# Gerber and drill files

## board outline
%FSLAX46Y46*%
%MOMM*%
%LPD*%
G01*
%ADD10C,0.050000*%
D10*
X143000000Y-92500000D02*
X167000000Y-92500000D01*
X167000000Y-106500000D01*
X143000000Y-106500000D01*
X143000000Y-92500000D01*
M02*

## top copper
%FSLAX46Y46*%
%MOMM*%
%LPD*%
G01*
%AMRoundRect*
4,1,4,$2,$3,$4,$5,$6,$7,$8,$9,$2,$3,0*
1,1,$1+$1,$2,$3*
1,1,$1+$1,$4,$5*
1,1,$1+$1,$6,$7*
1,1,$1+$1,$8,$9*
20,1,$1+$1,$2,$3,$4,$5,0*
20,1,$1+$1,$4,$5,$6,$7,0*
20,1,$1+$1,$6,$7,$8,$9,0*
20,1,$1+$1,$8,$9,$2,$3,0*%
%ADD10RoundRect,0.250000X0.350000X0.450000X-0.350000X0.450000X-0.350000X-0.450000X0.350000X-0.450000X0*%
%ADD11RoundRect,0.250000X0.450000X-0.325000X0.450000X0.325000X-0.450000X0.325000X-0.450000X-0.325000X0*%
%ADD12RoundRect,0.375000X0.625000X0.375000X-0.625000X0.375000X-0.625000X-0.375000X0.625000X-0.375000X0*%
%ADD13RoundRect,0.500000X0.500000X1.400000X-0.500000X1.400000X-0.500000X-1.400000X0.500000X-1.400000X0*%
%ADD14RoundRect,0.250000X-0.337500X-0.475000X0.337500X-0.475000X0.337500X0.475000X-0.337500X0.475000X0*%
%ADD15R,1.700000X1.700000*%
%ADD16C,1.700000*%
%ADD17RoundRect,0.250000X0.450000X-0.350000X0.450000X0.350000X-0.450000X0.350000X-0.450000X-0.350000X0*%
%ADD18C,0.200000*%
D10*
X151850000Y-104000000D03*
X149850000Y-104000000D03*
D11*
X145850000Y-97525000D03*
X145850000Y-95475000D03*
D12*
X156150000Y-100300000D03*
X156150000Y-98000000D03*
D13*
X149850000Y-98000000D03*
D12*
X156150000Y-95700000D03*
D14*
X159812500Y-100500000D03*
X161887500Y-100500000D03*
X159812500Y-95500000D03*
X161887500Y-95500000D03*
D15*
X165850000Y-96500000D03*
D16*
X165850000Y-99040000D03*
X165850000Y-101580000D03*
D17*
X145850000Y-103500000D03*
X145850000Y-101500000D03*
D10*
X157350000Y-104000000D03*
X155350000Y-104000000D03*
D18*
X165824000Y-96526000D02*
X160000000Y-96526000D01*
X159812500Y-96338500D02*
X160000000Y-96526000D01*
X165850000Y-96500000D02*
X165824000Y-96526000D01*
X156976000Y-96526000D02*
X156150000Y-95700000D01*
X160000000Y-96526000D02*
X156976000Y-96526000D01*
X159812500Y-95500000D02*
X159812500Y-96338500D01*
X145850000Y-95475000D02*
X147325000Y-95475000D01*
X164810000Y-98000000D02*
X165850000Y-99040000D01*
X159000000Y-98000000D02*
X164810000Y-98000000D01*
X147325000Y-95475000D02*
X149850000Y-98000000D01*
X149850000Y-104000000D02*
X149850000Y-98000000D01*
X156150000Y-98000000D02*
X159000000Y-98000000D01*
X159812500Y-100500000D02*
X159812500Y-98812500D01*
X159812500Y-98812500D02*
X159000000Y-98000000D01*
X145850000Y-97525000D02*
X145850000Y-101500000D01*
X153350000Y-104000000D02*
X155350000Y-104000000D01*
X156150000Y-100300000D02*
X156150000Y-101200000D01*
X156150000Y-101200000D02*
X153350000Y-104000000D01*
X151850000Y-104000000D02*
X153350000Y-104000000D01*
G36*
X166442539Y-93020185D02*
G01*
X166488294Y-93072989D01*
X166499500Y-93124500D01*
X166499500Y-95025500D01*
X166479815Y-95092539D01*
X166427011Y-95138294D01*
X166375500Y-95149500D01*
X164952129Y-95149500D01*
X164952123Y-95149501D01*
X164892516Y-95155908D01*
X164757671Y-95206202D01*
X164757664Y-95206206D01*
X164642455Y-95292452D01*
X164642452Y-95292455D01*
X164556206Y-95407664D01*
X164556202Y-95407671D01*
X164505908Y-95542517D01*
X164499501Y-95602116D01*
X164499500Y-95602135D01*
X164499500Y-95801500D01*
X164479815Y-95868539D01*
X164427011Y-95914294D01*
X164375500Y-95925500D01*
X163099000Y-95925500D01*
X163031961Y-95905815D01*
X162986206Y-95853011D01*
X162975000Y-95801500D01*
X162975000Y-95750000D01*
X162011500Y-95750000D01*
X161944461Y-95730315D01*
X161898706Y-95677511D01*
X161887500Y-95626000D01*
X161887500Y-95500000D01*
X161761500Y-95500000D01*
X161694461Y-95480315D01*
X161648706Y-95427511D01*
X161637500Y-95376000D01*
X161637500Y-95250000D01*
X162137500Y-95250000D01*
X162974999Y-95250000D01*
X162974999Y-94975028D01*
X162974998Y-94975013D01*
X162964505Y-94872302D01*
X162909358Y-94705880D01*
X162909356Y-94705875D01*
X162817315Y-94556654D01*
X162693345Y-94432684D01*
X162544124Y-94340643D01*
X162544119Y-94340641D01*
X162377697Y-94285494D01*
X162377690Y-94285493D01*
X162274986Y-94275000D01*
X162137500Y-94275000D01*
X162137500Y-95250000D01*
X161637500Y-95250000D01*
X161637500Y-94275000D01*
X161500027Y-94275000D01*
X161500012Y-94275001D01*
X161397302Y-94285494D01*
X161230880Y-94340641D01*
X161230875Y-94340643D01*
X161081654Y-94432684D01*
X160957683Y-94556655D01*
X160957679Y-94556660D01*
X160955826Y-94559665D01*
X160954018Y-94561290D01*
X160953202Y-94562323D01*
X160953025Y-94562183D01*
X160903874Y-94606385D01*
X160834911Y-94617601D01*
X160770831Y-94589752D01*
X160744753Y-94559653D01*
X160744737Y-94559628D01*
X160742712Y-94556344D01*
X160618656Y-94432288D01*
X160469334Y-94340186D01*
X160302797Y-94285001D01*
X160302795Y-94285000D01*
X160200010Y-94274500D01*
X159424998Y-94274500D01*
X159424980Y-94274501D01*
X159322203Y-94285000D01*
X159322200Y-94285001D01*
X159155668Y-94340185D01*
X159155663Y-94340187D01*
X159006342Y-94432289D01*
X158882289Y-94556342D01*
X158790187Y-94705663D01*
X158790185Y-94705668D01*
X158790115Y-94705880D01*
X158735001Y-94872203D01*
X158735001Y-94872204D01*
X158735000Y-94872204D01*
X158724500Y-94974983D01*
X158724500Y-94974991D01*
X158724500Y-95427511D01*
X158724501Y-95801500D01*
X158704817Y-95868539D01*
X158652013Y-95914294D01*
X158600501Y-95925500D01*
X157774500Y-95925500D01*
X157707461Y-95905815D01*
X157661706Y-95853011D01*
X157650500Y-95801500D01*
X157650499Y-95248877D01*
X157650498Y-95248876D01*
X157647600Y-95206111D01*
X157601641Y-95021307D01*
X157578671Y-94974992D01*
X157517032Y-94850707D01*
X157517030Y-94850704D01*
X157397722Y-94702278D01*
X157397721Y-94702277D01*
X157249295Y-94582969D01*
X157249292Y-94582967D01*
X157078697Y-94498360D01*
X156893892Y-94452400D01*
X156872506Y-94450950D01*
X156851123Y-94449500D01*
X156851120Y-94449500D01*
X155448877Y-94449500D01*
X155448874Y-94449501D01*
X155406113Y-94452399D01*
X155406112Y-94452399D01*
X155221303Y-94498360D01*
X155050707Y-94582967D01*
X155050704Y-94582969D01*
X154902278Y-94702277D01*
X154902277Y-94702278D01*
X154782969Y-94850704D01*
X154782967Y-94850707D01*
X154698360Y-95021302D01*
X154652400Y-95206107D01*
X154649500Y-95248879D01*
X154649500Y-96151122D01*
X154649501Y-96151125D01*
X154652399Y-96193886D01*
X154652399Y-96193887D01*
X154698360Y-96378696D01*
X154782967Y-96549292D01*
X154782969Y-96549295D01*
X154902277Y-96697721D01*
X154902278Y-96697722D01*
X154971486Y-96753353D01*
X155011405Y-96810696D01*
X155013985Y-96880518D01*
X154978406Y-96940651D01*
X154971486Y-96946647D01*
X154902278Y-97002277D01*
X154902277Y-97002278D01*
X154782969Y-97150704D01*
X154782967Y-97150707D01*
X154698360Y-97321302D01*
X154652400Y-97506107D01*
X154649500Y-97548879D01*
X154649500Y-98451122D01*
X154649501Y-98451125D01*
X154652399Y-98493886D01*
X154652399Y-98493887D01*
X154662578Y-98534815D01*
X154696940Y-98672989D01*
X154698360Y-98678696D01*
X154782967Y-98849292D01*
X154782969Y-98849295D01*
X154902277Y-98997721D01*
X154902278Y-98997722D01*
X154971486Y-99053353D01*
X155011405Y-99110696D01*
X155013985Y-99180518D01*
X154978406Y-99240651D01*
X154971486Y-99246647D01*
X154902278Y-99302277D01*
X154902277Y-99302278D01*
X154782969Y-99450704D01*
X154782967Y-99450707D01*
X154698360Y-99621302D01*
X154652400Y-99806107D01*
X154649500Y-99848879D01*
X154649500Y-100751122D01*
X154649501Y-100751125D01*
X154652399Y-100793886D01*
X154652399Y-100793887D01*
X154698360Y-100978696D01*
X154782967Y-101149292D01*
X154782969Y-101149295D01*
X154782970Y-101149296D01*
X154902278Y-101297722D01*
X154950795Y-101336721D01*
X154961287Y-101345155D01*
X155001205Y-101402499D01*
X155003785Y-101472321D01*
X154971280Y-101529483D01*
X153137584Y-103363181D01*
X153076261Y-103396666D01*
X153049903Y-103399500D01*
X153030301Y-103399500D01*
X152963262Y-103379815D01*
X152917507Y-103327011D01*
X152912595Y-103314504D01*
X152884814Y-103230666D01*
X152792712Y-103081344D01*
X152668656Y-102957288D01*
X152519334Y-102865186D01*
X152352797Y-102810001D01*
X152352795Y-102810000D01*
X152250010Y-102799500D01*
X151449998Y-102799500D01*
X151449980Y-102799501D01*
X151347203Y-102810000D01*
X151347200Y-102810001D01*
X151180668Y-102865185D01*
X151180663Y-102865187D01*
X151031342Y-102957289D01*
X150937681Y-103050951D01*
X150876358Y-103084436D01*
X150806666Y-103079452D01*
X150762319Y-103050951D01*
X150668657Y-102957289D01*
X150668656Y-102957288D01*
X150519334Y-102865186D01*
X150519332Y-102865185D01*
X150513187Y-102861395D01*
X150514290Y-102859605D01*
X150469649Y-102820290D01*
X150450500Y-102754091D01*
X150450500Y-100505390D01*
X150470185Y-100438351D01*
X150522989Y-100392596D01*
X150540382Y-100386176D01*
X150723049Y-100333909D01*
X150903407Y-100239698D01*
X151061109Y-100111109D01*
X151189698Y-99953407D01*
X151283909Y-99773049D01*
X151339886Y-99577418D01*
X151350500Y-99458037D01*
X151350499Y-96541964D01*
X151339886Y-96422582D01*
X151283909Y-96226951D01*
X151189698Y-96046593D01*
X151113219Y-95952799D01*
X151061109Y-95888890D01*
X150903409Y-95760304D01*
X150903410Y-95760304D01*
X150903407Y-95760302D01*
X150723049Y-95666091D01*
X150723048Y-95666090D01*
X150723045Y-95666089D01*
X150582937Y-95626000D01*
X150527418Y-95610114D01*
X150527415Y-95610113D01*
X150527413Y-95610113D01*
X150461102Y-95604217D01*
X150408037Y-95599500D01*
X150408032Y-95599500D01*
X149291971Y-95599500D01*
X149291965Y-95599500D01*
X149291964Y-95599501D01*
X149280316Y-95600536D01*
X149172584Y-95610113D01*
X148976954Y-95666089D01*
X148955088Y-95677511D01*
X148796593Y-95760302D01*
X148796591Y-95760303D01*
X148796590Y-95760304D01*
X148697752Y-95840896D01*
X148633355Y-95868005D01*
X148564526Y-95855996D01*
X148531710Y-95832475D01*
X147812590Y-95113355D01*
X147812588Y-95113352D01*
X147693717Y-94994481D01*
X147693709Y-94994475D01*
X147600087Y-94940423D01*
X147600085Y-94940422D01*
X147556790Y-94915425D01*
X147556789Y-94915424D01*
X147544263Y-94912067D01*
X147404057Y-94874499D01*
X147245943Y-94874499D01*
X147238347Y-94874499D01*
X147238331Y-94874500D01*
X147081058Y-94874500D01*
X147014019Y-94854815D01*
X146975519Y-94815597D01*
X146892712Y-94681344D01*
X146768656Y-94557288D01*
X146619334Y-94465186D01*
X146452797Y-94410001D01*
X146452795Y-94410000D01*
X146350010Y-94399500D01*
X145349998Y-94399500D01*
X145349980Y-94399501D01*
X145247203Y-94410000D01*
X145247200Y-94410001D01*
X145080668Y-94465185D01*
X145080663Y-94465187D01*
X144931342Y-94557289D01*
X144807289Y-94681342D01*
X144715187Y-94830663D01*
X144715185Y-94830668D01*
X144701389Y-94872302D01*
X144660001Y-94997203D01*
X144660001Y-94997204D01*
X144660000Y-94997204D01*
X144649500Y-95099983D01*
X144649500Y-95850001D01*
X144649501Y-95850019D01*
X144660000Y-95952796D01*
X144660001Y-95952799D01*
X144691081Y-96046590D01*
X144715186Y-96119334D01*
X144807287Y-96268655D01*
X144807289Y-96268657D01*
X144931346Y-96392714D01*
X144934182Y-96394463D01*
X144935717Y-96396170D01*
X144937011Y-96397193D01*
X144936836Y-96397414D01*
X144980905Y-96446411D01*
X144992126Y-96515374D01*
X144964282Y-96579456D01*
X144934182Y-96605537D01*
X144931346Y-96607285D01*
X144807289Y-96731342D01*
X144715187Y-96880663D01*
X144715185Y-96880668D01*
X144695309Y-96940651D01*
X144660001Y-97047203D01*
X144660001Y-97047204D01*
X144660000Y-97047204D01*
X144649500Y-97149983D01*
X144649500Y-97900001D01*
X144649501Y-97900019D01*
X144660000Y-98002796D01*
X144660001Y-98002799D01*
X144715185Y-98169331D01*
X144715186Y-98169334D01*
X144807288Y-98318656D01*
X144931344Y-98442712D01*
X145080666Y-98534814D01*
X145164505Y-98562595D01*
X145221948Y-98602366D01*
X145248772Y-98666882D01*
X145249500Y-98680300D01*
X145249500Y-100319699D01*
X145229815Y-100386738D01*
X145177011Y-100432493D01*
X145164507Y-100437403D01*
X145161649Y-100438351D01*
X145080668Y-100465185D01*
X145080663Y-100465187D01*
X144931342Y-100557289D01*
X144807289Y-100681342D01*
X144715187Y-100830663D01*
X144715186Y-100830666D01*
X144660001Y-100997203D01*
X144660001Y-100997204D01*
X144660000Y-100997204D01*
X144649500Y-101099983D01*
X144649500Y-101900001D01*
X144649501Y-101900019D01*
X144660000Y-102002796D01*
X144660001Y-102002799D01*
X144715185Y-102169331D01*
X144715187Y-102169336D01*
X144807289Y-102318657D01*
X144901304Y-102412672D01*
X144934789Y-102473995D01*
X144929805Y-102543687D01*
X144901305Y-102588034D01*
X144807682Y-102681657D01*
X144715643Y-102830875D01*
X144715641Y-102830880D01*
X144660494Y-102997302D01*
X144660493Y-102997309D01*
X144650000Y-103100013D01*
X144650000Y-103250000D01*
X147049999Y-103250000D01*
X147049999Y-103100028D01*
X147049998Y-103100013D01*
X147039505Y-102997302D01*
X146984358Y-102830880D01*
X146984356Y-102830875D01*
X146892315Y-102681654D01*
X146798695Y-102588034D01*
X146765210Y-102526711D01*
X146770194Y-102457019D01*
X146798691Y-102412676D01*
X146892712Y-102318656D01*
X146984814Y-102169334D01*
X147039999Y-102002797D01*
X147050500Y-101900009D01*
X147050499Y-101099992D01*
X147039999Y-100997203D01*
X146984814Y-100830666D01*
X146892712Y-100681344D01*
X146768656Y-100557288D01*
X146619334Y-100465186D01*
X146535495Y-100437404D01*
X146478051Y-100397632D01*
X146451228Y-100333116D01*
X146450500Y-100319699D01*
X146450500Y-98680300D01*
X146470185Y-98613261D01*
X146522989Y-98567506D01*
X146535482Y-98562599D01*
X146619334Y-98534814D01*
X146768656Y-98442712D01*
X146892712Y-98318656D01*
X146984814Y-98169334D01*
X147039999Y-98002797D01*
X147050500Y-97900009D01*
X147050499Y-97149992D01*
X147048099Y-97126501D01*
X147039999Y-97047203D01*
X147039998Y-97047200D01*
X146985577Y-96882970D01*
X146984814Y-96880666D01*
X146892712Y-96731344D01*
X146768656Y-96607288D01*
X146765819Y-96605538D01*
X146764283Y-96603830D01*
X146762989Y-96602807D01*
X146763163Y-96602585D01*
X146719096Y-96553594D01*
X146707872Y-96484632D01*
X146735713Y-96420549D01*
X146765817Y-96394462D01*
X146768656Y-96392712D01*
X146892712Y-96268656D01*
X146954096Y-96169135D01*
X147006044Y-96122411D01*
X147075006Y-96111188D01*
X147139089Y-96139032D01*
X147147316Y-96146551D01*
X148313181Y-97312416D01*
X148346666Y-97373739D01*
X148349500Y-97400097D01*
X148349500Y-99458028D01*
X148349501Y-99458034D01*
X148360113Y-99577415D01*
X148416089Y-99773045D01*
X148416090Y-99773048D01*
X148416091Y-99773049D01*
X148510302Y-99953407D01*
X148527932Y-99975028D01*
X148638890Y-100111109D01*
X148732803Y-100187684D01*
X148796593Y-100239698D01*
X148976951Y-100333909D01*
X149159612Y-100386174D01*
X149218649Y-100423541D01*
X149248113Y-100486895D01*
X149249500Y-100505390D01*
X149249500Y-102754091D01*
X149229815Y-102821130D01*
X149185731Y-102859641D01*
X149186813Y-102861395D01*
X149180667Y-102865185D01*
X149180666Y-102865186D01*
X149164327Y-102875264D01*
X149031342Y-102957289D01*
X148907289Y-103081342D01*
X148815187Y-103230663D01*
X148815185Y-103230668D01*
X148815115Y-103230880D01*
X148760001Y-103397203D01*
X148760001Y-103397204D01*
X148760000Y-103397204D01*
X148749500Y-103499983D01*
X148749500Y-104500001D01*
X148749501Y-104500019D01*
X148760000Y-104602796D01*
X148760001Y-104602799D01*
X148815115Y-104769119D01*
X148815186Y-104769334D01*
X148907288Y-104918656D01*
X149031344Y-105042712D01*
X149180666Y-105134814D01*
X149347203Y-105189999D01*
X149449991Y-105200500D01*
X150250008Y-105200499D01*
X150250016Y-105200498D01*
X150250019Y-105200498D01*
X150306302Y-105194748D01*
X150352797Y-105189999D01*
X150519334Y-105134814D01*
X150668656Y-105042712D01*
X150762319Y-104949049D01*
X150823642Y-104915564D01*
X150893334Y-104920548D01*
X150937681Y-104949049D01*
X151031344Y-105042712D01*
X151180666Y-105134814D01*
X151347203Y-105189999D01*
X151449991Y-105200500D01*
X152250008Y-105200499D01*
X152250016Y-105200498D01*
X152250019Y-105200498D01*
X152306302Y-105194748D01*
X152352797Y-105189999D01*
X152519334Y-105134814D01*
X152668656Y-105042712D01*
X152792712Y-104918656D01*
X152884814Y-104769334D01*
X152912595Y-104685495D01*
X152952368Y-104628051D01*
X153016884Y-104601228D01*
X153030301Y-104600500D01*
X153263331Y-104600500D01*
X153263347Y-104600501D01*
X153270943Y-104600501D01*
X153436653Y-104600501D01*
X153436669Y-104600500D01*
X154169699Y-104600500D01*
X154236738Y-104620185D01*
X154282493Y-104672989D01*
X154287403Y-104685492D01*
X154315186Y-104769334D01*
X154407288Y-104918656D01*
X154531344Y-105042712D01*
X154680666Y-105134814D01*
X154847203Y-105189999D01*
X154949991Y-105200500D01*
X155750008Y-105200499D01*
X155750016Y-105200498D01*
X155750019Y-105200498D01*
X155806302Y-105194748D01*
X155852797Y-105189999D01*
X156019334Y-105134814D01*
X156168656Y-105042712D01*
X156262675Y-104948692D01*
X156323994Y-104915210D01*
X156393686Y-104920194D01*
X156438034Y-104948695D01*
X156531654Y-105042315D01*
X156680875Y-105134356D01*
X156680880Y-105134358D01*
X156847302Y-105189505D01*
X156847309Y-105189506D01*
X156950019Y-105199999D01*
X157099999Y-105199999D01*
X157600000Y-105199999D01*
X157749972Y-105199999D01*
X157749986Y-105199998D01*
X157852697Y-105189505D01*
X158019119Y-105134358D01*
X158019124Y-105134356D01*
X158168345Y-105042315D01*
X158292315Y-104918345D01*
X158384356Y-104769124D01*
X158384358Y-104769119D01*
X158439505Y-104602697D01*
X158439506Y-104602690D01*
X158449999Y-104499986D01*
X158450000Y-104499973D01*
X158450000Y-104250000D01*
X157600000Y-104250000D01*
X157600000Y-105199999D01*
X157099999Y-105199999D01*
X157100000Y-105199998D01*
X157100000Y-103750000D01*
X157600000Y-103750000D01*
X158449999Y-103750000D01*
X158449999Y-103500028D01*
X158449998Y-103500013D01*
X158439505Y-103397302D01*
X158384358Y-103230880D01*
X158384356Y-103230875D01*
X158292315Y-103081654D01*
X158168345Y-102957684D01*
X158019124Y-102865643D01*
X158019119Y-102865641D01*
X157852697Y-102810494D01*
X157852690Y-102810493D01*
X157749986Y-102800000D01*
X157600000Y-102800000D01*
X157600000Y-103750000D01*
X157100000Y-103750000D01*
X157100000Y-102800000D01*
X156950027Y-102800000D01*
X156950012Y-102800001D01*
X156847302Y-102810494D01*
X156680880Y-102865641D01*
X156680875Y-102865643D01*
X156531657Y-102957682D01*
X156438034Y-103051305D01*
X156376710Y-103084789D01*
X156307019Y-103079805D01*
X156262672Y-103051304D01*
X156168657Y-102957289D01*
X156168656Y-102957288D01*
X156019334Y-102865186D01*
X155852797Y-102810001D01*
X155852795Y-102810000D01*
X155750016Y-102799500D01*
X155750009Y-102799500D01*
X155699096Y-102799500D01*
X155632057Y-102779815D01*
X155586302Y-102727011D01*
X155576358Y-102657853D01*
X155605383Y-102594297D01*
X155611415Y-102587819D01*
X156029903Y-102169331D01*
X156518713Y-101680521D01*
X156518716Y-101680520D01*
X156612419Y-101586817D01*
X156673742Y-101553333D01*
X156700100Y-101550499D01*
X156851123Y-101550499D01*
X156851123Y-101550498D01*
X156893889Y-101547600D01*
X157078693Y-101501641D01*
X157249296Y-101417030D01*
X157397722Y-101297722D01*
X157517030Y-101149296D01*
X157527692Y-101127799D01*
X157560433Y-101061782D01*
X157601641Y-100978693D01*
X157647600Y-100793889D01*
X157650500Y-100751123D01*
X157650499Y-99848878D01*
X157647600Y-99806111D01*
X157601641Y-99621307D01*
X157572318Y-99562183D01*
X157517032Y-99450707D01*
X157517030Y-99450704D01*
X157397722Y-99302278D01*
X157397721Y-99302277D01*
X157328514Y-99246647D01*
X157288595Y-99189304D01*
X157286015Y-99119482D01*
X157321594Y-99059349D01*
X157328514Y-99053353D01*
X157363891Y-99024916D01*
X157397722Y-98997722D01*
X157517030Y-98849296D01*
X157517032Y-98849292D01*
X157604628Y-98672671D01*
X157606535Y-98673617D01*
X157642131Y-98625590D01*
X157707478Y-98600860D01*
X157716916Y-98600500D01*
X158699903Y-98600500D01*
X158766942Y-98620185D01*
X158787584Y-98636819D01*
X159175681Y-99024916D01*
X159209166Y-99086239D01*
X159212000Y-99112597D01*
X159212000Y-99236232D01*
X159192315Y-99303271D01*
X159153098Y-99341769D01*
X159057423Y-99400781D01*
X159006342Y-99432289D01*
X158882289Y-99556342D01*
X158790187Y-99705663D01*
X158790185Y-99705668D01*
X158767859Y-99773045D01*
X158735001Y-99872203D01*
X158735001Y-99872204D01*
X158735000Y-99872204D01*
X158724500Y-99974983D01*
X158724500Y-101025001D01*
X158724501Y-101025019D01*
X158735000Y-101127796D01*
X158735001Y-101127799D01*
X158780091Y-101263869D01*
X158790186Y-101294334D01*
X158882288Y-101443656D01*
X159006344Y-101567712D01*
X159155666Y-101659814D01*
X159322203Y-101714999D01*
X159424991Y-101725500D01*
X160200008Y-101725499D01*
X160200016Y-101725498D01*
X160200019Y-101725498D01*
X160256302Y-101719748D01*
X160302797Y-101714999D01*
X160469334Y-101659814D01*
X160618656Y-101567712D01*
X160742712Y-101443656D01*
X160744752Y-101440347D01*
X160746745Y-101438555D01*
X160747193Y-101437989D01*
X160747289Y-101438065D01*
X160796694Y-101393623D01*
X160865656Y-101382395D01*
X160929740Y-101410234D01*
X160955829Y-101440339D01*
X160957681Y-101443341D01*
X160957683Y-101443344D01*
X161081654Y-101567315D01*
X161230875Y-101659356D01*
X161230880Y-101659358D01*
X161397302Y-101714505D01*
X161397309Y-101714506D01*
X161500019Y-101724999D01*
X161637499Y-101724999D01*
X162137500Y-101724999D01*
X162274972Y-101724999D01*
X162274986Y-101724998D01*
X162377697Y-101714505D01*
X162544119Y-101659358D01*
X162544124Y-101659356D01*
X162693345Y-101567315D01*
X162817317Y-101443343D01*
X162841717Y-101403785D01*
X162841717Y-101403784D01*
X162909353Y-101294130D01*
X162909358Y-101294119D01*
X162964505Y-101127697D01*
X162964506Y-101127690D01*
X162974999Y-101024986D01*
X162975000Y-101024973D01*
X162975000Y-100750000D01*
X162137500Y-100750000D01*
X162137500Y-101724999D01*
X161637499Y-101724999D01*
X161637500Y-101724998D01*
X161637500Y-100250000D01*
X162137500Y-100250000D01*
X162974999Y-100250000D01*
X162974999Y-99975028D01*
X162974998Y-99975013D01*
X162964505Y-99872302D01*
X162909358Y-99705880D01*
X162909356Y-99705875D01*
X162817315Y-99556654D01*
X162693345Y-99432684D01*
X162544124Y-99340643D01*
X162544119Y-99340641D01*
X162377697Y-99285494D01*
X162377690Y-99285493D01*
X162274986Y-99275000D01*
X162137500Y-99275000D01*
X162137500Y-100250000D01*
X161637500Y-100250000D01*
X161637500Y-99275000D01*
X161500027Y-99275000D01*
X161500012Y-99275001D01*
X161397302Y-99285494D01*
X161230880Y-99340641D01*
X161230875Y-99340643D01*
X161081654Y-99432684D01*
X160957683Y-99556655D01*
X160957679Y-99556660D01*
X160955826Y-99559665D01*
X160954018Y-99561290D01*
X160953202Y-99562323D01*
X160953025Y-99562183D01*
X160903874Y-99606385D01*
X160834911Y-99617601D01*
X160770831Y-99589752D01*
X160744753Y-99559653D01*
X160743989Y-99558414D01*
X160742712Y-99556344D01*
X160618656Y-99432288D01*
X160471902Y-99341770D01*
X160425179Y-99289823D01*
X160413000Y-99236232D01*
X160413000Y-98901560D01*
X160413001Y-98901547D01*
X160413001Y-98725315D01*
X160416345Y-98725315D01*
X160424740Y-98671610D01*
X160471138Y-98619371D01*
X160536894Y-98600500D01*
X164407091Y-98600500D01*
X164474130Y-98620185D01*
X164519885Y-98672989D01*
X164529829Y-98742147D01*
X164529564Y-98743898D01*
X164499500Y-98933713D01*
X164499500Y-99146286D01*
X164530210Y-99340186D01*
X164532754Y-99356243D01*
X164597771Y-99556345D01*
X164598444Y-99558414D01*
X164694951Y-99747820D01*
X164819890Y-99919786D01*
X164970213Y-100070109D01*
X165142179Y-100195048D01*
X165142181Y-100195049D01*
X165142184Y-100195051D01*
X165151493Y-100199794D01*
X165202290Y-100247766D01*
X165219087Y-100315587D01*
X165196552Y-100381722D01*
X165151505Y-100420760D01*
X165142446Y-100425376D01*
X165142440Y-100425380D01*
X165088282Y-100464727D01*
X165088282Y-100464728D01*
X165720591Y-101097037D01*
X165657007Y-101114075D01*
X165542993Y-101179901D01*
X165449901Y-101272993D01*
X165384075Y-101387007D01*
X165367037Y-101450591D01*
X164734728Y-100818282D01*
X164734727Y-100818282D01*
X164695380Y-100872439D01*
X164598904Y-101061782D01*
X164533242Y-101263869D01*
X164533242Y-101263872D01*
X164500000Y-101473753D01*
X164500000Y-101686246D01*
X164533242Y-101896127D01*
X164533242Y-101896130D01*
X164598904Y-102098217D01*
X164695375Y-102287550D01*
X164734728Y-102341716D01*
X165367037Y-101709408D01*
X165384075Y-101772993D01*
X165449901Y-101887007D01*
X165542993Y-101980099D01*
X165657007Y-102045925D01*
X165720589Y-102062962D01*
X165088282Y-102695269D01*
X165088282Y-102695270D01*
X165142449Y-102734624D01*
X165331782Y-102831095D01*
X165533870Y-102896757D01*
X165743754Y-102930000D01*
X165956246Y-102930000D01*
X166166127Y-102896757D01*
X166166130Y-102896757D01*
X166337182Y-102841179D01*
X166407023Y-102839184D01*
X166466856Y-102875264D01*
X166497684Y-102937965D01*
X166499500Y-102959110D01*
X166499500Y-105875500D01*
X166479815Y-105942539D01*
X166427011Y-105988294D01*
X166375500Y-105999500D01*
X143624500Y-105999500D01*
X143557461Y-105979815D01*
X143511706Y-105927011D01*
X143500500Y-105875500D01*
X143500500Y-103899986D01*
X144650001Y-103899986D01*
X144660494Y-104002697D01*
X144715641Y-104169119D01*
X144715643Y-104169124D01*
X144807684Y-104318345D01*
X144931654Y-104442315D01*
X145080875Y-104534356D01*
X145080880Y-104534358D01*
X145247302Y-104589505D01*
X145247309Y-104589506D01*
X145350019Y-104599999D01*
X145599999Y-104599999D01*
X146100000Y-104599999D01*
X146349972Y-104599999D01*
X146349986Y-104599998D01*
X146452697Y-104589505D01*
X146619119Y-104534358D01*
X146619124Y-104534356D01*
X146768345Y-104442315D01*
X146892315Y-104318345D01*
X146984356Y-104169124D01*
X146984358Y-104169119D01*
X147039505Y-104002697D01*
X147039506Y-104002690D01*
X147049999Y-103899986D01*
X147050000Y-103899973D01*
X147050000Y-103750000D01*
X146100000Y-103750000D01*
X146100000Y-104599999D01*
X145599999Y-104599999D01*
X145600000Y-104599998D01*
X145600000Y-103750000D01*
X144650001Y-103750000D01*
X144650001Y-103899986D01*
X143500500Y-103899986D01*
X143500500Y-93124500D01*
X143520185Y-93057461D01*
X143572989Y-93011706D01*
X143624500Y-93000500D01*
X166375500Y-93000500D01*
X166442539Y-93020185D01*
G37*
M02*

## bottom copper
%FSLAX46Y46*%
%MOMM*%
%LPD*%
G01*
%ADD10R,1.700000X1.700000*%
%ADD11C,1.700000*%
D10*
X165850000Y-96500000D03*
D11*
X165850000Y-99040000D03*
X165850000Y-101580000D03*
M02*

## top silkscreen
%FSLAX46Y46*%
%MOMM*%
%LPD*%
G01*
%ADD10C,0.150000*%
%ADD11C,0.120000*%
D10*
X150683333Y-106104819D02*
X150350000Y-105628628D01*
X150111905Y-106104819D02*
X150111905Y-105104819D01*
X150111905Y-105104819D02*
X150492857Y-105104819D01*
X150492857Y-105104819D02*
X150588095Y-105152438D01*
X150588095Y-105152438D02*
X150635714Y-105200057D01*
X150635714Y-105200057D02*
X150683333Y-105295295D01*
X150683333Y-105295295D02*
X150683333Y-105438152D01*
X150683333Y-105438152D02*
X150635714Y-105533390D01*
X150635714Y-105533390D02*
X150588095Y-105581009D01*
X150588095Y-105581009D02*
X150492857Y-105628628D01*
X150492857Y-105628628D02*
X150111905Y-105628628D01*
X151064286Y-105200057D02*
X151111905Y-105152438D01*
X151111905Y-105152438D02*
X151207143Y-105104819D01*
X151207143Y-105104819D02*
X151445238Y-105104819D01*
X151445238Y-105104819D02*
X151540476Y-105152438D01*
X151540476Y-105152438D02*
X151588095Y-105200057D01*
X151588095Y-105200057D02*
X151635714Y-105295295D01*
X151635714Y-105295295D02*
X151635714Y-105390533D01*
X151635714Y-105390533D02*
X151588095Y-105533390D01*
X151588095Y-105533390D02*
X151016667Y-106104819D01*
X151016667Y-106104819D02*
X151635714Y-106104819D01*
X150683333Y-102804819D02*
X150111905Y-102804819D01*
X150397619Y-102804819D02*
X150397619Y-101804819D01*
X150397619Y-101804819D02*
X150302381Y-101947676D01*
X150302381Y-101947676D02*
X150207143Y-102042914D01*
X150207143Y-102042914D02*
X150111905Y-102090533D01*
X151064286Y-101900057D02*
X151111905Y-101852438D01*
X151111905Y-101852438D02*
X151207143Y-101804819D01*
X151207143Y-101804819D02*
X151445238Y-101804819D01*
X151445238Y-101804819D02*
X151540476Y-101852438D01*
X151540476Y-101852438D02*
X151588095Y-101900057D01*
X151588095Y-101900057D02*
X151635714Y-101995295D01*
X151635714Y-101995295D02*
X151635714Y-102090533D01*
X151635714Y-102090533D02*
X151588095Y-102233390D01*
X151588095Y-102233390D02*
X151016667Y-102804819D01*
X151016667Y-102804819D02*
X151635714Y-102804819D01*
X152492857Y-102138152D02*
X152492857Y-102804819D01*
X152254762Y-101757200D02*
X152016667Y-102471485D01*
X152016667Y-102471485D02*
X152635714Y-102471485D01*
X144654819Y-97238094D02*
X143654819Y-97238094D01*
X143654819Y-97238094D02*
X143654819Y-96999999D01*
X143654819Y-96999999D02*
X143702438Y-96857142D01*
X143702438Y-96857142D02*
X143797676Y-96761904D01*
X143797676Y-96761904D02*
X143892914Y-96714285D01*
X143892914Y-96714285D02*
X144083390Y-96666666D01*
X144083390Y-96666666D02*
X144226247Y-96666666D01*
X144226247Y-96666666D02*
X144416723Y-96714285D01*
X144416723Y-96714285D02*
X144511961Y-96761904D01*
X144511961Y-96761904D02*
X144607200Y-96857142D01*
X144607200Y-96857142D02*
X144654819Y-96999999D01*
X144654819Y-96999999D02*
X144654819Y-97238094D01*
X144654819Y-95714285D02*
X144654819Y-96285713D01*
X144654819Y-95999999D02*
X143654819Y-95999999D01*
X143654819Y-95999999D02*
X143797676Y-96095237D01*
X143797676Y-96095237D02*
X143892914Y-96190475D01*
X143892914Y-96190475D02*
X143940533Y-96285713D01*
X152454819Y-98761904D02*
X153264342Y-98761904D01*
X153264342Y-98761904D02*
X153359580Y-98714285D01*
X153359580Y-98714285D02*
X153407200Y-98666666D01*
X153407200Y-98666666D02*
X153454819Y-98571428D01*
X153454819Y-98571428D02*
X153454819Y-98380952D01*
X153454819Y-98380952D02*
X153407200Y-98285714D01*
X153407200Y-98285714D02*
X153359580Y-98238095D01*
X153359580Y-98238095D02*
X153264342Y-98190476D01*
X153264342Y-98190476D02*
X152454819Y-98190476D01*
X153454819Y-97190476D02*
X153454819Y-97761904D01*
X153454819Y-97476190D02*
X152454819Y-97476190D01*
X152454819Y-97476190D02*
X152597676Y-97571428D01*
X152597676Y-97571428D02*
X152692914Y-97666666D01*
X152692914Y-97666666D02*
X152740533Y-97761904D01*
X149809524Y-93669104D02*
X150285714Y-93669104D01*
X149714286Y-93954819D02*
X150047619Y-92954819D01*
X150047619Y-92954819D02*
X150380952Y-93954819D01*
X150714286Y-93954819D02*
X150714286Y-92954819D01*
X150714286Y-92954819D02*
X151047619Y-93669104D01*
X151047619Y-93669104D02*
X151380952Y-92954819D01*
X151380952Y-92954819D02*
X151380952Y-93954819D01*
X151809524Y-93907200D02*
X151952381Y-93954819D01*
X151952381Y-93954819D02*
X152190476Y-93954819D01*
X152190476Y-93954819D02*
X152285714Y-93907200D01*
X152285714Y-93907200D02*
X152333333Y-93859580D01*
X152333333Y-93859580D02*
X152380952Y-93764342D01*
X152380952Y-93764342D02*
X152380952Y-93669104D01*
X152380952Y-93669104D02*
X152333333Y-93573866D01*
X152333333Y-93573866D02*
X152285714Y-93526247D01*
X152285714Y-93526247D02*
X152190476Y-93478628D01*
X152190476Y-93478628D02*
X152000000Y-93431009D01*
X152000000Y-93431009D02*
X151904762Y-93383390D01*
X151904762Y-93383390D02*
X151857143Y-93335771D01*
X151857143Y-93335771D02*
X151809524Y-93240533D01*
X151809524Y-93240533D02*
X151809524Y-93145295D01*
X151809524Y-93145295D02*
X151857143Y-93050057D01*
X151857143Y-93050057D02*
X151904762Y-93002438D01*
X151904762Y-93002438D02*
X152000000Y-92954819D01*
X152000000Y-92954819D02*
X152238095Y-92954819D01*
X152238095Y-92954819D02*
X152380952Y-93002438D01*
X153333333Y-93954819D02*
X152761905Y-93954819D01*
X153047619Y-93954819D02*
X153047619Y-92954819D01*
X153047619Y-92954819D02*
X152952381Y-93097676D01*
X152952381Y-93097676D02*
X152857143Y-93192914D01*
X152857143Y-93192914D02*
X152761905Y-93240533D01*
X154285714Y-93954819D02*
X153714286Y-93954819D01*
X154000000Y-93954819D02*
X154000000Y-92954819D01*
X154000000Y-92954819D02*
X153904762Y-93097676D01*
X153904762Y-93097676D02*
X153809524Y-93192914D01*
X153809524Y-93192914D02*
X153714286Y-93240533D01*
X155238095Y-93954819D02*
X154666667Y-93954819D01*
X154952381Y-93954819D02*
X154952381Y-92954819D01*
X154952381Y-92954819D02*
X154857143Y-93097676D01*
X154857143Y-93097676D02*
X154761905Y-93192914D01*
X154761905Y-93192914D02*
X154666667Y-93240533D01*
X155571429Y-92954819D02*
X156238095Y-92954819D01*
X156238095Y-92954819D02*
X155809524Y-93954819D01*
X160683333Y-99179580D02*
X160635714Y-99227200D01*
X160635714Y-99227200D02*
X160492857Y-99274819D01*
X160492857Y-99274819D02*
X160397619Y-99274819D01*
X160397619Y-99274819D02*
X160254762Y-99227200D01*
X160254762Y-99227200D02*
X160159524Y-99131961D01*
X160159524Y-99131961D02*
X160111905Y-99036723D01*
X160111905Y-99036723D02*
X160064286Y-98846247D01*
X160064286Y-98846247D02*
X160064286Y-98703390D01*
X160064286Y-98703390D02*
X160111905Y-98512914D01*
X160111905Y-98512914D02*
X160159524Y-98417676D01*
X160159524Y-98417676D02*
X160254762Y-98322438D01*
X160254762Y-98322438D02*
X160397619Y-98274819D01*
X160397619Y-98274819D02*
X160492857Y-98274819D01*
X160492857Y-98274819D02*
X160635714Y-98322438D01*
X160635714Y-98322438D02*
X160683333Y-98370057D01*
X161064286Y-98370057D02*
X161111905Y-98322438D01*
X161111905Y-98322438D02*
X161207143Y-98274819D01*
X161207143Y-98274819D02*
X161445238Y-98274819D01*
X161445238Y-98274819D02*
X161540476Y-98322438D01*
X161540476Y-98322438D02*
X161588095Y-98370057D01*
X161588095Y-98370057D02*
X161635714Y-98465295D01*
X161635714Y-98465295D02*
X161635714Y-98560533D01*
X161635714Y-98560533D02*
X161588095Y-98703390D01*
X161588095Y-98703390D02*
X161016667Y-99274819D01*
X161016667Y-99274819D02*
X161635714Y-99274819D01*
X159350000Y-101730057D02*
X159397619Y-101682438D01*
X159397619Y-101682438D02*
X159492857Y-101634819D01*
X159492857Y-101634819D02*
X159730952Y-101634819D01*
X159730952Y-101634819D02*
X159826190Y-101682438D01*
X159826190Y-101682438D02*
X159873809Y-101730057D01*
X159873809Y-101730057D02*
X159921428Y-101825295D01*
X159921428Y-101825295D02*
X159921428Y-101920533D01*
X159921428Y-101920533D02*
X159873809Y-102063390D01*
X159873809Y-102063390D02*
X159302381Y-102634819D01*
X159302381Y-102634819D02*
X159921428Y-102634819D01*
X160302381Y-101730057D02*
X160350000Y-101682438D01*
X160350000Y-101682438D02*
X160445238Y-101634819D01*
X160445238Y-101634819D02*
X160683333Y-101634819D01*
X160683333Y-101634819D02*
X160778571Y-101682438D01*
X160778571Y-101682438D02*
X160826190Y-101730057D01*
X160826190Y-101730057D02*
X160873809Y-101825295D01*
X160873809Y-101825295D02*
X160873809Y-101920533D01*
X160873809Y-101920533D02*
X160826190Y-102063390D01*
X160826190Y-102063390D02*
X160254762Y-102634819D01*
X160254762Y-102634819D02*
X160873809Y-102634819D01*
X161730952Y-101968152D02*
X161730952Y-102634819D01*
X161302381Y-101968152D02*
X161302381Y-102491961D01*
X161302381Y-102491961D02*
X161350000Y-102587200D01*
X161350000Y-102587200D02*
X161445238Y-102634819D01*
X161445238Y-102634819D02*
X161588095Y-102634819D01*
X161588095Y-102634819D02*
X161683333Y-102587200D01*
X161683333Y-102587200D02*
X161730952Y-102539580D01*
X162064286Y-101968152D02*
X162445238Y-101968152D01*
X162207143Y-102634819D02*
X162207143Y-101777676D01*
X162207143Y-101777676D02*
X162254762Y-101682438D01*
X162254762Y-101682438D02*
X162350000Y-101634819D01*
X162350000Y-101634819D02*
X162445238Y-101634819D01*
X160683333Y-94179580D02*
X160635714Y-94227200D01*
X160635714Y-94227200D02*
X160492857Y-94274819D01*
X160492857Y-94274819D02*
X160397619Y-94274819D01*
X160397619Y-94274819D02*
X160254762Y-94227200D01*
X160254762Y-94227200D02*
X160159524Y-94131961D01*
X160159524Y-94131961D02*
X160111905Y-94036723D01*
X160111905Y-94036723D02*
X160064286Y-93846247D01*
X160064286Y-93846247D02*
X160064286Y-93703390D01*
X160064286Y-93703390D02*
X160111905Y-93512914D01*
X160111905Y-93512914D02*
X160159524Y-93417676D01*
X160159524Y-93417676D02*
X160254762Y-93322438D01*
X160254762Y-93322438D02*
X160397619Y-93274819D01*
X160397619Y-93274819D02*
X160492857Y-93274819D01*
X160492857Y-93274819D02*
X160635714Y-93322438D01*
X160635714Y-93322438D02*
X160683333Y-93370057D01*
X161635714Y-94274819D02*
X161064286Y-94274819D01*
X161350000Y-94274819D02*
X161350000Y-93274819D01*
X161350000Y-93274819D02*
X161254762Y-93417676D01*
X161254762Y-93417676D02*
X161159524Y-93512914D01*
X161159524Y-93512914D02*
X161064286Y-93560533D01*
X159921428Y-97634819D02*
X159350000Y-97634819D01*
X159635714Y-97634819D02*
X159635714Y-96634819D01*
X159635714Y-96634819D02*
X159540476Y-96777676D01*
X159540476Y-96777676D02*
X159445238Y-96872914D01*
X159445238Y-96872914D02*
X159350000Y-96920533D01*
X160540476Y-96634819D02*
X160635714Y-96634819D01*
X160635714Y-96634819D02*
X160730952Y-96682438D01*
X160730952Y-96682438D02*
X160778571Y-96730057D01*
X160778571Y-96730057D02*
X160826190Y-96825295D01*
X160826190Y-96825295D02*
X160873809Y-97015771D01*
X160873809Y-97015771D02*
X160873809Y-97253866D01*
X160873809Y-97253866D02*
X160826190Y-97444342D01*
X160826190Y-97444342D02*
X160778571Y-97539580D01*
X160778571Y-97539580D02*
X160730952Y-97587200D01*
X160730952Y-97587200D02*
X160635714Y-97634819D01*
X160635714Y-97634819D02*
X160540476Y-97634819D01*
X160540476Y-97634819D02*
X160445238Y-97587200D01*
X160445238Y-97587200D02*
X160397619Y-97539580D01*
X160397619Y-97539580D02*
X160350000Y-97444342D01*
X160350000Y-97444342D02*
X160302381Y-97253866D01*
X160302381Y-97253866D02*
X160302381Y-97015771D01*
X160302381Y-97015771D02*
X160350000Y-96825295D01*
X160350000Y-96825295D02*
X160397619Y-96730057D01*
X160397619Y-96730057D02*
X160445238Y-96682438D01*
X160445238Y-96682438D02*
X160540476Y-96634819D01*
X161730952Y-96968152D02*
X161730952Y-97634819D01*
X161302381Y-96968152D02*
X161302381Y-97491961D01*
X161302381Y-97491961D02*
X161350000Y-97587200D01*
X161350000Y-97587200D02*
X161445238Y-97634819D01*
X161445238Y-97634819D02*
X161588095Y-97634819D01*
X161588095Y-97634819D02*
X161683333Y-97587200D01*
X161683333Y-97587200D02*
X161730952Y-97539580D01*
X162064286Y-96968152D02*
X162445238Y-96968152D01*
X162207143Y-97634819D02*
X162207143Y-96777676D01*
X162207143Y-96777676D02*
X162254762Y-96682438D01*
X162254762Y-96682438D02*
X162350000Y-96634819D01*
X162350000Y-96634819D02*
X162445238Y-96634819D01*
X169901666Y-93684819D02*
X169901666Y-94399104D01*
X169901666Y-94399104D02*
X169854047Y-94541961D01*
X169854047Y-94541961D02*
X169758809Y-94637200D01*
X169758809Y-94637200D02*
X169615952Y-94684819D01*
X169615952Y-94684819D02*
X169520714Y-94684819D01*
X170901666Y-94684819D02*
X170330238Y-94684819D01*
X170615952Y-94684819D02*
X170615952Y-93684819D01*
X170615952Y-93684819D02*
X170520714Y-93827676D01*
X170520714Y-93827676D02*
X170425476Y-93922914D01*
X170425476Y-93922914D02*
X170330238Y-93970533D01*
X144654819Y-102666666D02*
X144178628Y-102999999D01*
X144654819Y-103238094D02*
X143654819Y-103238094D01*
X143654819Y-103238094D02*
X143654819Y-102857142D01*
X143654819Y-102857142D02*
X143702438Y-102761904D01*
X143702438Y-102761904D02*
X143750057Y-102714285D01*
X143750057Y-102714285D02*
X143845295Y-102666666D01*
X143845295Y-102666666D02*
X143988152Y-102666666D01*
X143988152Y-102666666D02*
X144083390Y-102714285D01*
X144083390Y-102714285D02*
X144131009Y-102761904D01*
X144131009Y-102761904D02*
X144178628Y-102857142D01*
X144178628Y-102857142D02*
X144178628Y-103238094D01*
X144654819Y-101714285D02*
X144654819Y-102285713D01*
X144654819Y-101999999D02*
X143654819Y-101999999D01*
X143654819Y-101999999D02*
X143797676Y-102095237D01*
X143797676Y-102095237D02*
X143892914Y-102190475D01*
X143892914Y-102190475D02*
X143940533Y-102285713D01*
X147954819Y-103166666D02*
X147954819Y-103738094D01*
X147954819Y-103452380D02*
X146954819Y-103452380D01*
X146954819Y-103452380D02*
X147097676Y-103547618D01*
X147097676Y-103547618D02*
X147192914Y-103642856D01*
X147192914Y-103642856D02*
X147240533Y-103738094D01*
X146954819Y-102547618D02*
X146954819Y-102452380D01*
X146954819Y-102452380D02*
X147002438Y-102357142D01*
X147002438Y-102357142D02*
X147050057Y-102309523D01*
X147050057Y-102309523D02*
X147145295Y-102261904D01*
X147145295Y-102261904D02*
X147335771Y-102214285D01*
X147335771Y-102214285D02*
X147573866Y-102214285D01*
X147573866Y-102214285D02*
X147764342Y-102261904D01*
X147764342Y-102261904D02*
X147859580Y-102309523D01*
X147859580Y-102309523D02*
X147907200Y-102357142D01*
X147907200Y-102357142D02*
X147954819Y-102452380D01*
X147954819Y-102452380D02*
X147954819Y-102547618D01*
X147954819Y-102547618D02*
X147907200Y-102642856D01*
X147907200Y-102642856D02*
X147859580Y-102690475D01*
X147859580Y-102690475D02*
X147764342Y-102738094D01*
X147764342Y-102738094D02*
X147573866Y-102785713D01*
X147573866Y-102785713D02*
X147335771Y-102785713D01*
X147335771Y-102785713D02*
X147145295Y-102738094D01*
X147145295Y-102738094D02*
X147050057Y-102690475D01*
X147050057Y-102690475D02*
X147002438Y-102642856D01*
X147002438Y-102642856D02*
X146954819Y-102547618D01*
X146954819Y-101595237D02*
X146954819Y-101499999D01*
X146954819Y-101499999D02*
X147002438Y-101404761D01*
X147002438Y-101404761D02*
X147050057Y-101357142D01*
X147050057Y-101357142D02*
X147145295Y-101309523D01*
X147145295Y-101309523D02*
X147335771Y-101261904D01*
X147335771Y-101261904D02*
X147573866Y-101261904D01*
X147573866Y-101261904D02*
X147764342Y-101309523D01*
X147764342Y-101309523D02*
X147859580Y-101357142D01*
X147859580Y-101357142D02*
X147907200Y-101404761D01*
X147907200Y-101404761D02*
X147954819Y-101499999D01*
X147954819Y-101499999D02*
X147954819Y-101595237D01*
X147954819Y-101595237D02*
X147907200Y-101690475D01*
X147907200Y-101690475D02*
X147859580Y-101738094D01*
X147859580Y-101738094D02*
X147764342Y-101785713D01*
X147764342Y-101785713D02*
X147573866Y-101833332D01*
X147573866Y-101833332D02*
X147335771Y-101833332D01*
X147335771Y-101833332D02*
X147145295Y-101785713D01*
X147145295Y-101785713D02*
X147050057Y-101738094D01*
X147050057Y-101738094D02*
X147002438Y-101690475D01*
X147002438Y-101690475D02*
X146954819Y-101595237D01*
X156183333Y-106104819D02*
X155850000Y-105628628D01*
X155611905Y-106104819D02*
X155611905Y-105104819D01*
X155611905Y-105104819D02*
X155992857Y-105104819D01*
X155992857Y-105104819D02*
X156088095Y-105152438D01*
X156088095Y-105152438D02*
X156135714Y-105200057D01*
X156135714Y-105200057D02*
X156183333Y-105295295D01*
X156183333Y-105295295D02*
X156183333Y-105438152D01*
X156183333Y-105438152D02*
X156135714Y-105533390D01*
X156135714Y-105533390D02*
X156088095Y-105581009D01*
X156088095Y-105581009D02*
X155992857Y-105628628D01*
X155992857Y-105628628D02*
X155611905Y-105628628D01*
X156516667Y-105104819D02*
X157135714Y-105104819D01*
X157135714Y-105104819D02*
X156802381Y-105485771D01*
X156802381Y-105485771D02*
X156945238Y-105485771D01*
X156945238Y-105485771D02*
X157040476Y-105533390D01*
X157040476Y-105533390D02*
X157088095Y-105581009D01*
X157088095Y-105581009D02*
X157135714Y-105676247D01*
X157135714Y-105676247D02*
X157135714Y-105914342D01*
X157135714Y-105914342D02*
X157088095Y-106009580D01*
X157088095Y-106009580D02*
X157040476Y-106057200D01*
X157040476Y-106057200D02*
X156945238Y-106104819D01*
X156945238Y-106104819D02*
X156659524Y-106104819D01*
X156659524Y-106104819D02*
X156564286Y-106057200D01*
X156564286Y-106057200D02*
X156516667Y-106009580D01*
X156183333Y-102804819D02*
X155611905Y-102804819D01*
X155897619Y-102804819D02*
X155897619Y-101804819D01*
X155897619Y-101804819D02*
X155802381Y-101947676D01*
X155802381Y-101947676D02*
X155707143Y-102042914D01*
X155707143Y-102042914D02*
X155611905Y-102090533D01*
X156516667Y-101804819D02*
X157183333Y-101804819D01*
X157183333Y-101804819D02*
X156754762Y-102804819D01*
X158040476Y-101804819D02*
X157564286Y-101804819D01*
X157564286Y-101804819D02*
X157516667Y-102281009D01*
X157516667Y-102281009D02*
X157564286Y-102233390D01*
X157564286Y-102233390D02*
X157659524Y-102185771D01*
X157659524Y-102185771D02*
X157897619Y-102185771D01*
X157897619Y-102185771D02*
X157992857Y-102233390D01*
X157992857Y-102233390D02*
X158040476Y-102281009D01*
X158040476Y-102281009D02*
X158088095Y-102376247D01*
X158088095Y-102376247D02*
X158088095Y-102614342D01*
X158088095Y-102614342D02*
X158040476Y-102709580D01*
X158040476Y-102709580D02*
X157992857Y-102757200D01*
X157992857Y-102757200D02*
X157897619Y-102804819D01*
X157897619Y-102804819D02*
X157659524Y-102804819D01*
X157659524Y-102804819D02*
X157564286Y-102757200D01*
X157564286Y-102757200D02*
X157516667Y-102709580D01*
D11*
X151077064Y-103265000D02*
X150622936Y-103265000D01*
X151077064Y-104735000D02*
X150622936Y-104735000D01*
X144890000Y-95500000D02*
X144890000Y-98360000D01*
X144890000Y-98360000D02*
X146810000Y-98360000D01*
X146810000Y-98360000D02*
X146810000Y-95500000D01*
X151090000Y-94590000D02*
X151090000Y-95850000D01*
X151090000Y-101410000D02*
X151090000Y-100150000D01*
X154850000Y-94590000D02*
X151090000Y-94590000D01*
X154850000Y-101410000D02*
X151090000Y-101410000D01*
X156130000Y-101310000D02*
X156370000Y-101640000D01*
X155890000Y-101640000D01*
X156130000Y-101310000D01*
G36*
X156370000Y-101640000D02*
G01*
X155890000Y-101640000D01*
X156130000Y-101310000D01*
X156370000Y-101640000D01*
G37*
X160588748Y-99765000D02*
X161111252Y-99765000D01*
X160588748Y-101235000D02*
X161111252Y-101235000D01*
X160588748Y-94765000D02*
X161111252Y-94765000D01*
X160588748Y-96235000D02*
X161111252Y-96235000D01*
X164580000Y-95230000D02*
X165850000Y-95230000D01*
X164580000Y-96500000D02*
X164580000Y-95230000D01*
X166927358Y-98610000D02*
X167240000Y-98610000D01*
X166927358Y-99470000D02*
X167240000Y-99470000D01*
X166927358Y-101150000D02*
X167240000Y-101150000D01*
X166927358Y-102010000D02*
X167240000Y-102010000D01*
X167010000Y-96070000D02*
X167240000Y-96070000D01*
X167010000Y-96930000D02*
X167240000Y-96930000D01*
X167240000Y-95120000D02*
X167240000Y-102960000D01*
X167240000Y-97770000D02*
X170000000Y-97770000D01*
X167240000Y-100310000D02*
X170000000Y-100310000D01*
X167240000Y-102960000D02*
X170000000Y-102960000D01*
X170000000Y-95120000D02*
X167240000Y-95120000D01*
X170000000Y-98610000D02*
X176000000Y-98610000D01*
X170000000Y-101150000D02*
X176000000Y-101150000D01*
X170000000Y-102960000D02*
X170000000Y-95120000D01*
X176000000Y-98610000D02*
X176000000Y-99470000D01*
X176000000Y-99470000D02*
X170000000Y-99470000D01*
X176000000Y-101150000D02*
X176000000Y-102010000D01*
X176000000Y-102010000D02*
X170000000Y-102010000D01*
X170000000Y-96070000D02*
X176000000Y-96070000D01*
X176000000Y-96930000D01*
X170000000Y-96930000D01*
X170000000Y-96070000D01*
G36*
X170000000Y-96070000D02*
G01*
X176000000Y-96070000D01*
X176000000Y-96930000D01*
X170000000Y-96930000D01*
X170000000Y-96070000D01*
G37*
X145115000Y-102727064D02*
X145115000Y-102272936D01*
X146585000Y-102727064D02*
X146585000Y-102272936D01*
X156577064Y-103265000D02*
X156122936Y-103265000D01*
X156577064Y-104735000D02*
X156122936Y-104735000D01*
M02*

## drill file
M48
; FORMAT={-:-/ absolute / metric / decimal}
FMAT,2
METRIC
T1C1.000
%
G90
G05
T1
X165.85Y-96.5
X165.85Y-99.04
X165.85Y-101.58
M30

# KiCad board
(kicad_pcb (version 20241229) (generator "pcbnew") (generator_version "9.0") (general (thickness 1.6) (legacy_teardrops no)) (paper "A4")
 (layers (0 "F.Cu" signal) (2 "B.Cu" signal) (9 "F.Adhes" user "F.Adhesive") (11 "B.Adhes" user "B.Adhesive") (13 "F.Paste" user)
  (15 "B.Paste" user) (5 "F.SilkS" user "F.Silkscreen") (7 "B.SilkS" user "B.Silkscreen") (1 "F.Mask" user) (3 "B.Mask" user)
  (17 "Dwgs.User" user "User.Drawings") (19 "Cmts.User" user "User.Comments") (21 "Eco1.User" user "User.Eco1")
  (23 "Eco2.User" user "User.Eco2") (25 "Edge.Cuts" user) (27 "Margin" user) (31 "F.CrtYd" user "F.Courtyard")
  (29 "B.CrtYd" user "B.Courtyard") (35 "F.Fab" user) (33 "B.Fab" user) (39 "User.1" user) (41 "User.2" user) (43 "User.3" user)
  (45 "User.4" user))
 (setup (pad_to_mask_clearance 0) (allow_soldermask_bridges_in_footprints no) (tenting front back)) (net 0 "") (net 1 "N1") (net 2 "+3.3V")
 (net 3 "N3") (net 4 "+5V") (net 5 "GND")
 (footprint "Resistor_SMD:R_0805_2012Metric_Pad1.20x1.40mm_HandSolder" (layer "F.Cu") (at 150.85 104 180)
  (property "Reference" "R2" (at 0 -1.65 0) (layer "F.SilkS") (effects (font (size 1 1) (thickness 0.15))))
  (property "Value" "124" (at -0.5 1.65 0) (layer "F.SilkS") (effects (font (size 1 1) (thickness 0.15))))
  (fp_line (start -0.227064 0.735) (end 0.227064 0.735) (stroke (width 0.12) (type solid)) (layer "F.SilkS"))
  (fp_line (start -0.227064 -0.735) (end 0.227064 -0.735) (stroke (width 0.12) (type solid)) (layer "F.SilkS"))
  (pad "1" smd roundrect (at -1 0 180) (size 1.2 1.4) (layers "F.Cu" "F.Mask" "F.Paste") (roundrect_rratio 0.208333) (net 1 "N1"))
  (pad "2" smd roundrect (at 1 0 180) (size 1.2 1.4) (layers "F.Cu" "F.Mask" "F.Paste") (roundrect_rratio 0.208333) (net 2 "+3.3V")))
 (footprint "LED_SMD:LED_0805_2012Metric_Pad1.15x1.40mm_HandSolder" (layer "F.Cu") (at 145.85 96.5 90)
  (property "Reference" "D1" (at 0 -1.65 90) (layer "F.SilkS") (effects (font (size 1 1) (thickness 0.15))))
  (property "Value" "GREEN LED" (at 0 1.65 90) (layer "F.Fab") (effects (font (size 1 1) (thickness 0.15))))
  (fp_line (start 1 -0.96) (end -1.86 -0.96) (stroke (width 0.12) (type solid)) (layer "F.SilkS"))
  (fp_line (start -1.86 -0.96) (end -1.86 0.96) (stroke (width 0.12) (type solid)) (layer "F.SilkS"))
  (fp_line (start -1.86 0.96) (end 1 0.96) (stroke (width 0.12) (type solid)) (layer "F.SilkS"))
  (pad "1" smd roundrect (at -1.025 0 90) (size 1.15 1.4) (layers "F.Cu" "F.Mask" "F.Paste") (roundrect_rratio 0.217391) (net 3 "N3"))
  (pad "2" smd roundrect (at 1.025 0 90) (size 1.15 1.4) (layers "F.Cu" "F.Mask" "F.Paste") (roundrect_rratio 0.217391) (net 2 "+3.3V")))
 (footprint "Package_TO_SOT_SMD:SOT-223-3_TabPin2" (layer "F.Cu") (at 153 98 180)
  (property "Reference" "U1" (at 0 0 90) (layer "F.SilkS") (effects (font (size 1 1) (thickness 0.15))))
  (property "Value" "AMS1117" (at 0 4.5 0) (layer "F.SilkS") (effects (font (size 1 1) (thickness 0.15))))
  (fp_line (start 1.91 3.41) (end 1.91 2.15) (stroke (width 0.12) (type solid)) (layer "F.SilkS"))
  (fp_line (start 1.91 -3.41) (end 1.91 -2.15) (stroke (width 0.12) (type solid)) (layer "F.SilkS"))
  (fp_line (start -1.85 3.41) (end 1.91 3.41) (stroke (width 0.12) (type solid)) (layer "F.SilkS"))
  (fp_line (start -1.85 -3.41) (end 1.91 -3.41) (stroke (width 0.12) (type solid)) (layer "F.SilkS"))
  (fp_poly
   (pts (xy -3.13 -3.31) (xy -3.37 -3.64) (xy -2.89 -3.64) (xy -3.13 -3.31)) (stroke (width 0.12) (type solid)) (fill yes) (layer "F.SilkS"))
  (pad "1" smd roundrect (at -3.15 -2.3 180) (size 2 1.5) (layers "F.Cu" "F.Mask" "F.Paste") (roundrect_rratio 0.25) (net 1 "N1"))
  (pad "2" smd roundrect (at -3.15 0 180) (size 2 1.5) (layers "F.Cu" "F.Mask" "F.Paste") (roundrect_rratio 0.25) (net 2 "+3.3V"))
  (pad "2" smd roundrect (at 3.15 0 180) (size 2 3.8) (layers "F.Cu" "F.Mask" "F.Paste") (roundrect_rratio 0.25) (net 2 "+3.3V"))
  (pad "3" smd roundrect (at -3.15 2.3 180) (size 2 1.5) (layers "F.Cu" "F.Mask" "F.Paste") (roundrect_rratio 0.25) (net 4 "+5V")))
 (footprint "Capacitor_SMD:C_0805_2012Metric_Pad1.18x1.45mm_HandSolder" (layer "F.Cu") (at 160.85 100.5)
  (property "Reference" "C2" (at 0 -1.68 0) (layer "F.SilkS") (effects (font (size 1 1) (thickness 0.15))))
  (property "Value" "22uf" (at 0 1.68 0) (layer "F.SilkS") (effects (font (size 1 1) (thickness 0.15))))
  (fp_line (start -0.261252 -0.735) (end 0.261252 -0.735) (stroke (width 0.12) (type solid)) (layer "F.SilkS"))
  (fp_line (start -0.261252 0.735) (end 0.261252 0.735) (stroke (width 0.12) (type solid)) (layer "F.SilkS"))
  (pad "1" smd roundrect (at -1.0375 0) (size 1.175 1.45) (layers "F.Cu" "F.Mask" "F.Paste") (roundrect_rratio 0.212766) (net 2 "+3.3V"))
  (pad "2" smd roundrect (at 1.0375 0) (size 1.175 1.45) (layers "F.Cu" "F.Mask" "F.Paste") (roundrect_rratio 0.212766) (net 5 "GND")))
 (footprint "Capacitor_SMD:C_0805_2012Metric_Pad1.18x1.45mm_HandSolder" (layer "F.Cu") (at 160.85 95.5)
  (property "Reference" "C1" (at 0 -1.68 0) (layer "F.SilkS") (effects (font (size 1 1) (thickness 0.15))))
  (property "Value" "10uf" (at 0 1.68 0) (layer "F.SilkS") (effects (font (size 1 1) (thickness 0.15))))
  (fp_line (start -0.261252 -0.735) (end 0.261252 -0.735) (stroke (width 0.12) (type solid)) (layer "F.SilkS"))
  (fp_line (start -0.261252 0.735) (end 0.261252 0.735) (stroke (width 0.12) (type solid)) (layer "F.SilkS"))
  (pad "1" smd roundrect (at -1.0375 0) (size 1.175 1.45) (layers "F.Cu" "F.Mask" "F.Paste") (roundrect_rratio 0.212766) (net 4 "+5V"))
  (pad "2" smd roundrect (at 1.0375 0) (size 1.175 1.45) (layers "F.Cu" "F.Mask" "F.Paste") (roundrect_rratio 0.212766) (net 5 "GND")))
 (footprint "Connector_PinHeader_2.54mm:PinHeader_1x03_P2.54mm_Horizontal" (layer "F.Cu") (at 165.85 96.5)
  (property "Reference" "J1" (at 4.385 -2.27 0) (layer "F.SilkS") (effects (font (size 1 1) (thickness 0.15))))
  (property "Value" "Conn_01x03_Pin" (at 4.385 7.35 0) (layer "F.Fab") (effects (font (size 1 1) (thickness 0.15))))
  (fp_line (start -1.27 -1.27) (end 0 -1.27) (stroke (width 0.12) (type solid)) (layer "F.SilkS"))
  (fp_line (start -1.27 0) (end -1.27 -1.27) (stroke (width 0.12) (type solid)) (layer "F.SilkS"))
  (fp_line (start 1.077358 2.11) (end 1.39 2.11) (stroke (width 0.12) (type solid)) (layer "F.SilkS"))
  (fp_line (start 1.077358 2.97) (end 1.39 2.97) (stroke (width 0.12) (type solid)) (layer "F.SilkS"))
  (fp_line (start 1.077358 4.65) (end 1.39 4.65) (stroke (width 0.12) (type solid)) (layer "F.SilkS"))
  (fp_line (start 1.077358 5.51) (end 1.39 5.51) (stroke (width 0.12) (type solid)) (layer "F.SilkS"))
  (fp_line (start 1.16 -0.43) (end 1.39 -0.43) (stroke (width 0.12) (type solid)) (layer "F.SilkS"))
  (fp_line (start 1.16 0.43) (end 1.39 0.43) (stroke (width 0.12) (type solid)) (layer "F.SilkS"))
  (fp_line (start 1.39 -1.38) (end 1.39 6.46) (stroke (width 0.12) (type solid)) (layer "F.SilkS"))
  (fp_line (start 1.39 1.27) (end 4.15 1.27) (stroke (width 0.12) (type solid)) (layer "F.SilkS"))
  (fp_line (start 1.39 3.81) (end 4.15 3.81) (stroke (width 0.12) (type solid)) (layer "F.SilkS"))
  (fp_line (start 1.39 6.46) (end 4.15 6.46) (stroke (width 0.12) (type solid)) (layer "F.SilkS"))
  (fp_line (start 4.15 -1.38) (end 1.39 -1.38) (stroke (width 0.12) (type solid)) (layer "F.SilkS"))
  (fp_line (start 4.15 2.11) (end 10.15 2.11) (stroke (width 0.12) (type solid)) (layer "F.SilkS"))
  (fp_line (start 4.15 4.65) (end 10.15 4.65) (stroke (width 0.12) (type solid)) (layer "F.SilkS"))
  (fp_line (start 4.15 6.46) (end 4.15 -1.38) (stroke (width 0.12) (type solid)) (layer "F.SilkS"))
  (fp_line (start 10.15 2.11) (end 10.15 2.97) (stroke (width 0.12) (type solid)) (layer "F.SilkS"))
  (fp_line (start 10.15 2.97) (end 4.15 2.97) (stroke (width 0.12) (type solid)) (layer "F.SilkS"))
  (fp_line (start 10.15 4.65) (end 10.15 5.51) (stroke (width 0.12) (type solid)) (layer "F.SilkS"))
  (fp_line (start 10.15 5.51) (end 4.15 5.51) (stroke (width 0.12) (type solid)) (layer "F.SilkS"))
  (fp_rect (start 4.15 -0.43) (end 10.15 0.43) (stroke (width 0.12) (type solid)) (fill yes) (layer "F.SilkS"))
  (pad "1" thru_hole rect (at 0 0) (size 1.7 1.7) (drill 1) (layers "*.Cu" "*.Mask") (remove_unused_layers no) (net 4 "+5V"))
  (pad "2" thru_hole circle (at 0 2.54) (size 1.7 1.7) (drill 1) (layers "*.Cu" "*.Mask") (remove_unused_layers no) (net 2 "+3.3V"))
  (pad "3" thru_hole circle (at 0 5.08) (size 1.7 1.7) (drill 1) (layers "*.Cu" "*.Mask") (remove_unused_layers no) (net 5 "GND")))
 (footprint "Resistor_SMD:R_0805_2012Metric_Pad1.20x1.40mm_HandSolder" (layer "F.Cu") (at 145.85 102.5 90)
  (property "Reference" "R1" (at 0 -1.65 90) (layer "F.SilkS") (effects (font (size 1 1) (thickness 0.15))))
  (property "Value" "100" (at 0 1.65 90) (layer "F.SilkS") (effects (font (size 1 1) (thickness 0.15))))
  (fp_line (start -0.227064 -0.735) (end 0.227064 -0.735) (stroke (width 0.12) (type solid)) (layer "F.SilkS"))
  (fp_line (start -0.227064 0.735) (end 0.227064 0.735) (stroke (width 0.12) (type solid)) (layer "F.SilkS"))
  (pad "1" smd roundrect (at -1 0 90) (size 1.2 1.4) (layers "F.Cu" "F.Mask" "F.Paste") (roundrect_rratio 0.208333) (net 5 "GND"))
  (pad "2" smd roundrect (at 1 0 90) (size 1.2 1.4) (layers "F.Cu" "F.Mask" "F.Paste") (roundrect_rratio 0.208333) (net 3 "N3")))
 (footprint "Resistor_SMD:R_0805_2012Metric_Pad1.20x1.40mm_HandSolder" (layer "F.Cu") (at 156.35 104 180)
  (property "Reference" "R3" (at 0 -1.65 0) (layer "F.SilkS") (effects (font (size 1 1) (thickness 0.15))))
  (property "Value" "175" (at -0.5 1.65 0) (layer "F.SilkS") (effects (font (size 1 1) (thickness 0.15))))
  (fp_line (start -0.227064 0.735) (end 0.227064 0.735) (stroke (width 0.12) (type solid)) (layer "F.SilkS"))
  (fp_line (start -0.227064 -0.735) (end 0.227064 -0.735) (stroke (width 0.12) (type solid)) (layer "F.SilkS"))
  (pad "1" smd roundrect (at -1 0 180) (size 1.2 1.4) (layers "F.Cu" "F.Mask" "F.Paste") (roundrect_rratio 0.208333) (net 5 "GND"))
  (pad "2" smd roundrect (at 1 0 180) (size 1.2 1.4) (layers "F.Cu" "F.Mask" "F.Paste") (roundrect_rratio 0.208333) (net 1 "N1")))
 (gr_rect (start 143 92.5) (end 167 106.5) (stroke (width 0.05) (type default)) (fill no) (layer "Edge.Cuts"))
 (segment (start 165.824 96.526) (end 160 96.526) (width 0.2) (layer "F.Cu") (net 4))
 (segment (start 159.8125 96.3385) (end 160 96.526) (width 0.2) (layer "F.Cu") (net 4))
 (segment (start 165.85 96.5) (end 165.824 96.526) (width 0.2) (layer "F.Cu") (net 4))
 (segment (start 156.976 96.526) (end 156.15 95.7) (width 0.2) (layer "F.Cu") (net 4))
 (segment (start 160 96.526) (end 156.976 96.526) (width 0.2) (layer "F.Cu") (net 4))
 (segment (start 159.8125 95.5) (end 159.8125 96.3385) (width 0.2) (layer "F.Cu") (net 4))
 (segment (start 145.85 95.475) (end 147.325 95.475) (width 0.2) (layer "F.Cu") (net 2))
 (segment (start 164.81 98) (end 165.85 99.04) (width 0.2) (layer "F.Cu") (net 2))
 (segment (start 159 98) (end 164.81 98) (width 0.2) (layer "F.Cu") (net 2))
 (segment (start 147.325 95.475) (end 149.85 98) (width 0.2) (layer "F.Cu") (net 2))
 (segment (start 149.85 104) (end 149.85 98) (width 0.2) (layer "F.Cu") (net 2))
 (segment (start 156.15 98) (end 159 98) (width 0.2) (layer "F.Cu") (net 2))
 (segment (start 159.8125 100.5) (end 159.8125 98.8125) (width 0.2) (layer "F.Cu") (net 2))
 (segment (start 159.8125 98.8125) (end 159 98) (width 0.2) (layer "F.Cu") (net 2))
 (segment (start 145.85 97.525) (end 145.85 101.5) (width 0.2) (layer "F.Cu") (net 3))
 (segment (start 153.35 104) (end 155.35 104) (width 0.2) (layer "F.Cu") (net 1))
 (segment (start 156.15 100.3) (end 156.15 101.2) (width 0.2) (layer "F.Cu") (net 1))
 (segment (start 156.15 101.2) (end 153.35 104) (width 0.2) (layer "F.Cu") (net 1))
 (segment (start 151.85 104) (end 153.35 104) (width 0.2) (layer "F.Cu") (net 1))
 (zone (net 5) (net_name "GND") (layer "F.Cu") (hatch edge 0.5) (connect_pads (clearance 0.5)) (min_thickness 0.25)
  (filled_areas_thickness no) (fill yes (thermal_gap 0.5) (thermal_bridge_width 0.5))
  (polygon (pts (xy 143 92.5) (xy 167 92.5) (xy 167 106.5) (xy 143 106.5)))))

